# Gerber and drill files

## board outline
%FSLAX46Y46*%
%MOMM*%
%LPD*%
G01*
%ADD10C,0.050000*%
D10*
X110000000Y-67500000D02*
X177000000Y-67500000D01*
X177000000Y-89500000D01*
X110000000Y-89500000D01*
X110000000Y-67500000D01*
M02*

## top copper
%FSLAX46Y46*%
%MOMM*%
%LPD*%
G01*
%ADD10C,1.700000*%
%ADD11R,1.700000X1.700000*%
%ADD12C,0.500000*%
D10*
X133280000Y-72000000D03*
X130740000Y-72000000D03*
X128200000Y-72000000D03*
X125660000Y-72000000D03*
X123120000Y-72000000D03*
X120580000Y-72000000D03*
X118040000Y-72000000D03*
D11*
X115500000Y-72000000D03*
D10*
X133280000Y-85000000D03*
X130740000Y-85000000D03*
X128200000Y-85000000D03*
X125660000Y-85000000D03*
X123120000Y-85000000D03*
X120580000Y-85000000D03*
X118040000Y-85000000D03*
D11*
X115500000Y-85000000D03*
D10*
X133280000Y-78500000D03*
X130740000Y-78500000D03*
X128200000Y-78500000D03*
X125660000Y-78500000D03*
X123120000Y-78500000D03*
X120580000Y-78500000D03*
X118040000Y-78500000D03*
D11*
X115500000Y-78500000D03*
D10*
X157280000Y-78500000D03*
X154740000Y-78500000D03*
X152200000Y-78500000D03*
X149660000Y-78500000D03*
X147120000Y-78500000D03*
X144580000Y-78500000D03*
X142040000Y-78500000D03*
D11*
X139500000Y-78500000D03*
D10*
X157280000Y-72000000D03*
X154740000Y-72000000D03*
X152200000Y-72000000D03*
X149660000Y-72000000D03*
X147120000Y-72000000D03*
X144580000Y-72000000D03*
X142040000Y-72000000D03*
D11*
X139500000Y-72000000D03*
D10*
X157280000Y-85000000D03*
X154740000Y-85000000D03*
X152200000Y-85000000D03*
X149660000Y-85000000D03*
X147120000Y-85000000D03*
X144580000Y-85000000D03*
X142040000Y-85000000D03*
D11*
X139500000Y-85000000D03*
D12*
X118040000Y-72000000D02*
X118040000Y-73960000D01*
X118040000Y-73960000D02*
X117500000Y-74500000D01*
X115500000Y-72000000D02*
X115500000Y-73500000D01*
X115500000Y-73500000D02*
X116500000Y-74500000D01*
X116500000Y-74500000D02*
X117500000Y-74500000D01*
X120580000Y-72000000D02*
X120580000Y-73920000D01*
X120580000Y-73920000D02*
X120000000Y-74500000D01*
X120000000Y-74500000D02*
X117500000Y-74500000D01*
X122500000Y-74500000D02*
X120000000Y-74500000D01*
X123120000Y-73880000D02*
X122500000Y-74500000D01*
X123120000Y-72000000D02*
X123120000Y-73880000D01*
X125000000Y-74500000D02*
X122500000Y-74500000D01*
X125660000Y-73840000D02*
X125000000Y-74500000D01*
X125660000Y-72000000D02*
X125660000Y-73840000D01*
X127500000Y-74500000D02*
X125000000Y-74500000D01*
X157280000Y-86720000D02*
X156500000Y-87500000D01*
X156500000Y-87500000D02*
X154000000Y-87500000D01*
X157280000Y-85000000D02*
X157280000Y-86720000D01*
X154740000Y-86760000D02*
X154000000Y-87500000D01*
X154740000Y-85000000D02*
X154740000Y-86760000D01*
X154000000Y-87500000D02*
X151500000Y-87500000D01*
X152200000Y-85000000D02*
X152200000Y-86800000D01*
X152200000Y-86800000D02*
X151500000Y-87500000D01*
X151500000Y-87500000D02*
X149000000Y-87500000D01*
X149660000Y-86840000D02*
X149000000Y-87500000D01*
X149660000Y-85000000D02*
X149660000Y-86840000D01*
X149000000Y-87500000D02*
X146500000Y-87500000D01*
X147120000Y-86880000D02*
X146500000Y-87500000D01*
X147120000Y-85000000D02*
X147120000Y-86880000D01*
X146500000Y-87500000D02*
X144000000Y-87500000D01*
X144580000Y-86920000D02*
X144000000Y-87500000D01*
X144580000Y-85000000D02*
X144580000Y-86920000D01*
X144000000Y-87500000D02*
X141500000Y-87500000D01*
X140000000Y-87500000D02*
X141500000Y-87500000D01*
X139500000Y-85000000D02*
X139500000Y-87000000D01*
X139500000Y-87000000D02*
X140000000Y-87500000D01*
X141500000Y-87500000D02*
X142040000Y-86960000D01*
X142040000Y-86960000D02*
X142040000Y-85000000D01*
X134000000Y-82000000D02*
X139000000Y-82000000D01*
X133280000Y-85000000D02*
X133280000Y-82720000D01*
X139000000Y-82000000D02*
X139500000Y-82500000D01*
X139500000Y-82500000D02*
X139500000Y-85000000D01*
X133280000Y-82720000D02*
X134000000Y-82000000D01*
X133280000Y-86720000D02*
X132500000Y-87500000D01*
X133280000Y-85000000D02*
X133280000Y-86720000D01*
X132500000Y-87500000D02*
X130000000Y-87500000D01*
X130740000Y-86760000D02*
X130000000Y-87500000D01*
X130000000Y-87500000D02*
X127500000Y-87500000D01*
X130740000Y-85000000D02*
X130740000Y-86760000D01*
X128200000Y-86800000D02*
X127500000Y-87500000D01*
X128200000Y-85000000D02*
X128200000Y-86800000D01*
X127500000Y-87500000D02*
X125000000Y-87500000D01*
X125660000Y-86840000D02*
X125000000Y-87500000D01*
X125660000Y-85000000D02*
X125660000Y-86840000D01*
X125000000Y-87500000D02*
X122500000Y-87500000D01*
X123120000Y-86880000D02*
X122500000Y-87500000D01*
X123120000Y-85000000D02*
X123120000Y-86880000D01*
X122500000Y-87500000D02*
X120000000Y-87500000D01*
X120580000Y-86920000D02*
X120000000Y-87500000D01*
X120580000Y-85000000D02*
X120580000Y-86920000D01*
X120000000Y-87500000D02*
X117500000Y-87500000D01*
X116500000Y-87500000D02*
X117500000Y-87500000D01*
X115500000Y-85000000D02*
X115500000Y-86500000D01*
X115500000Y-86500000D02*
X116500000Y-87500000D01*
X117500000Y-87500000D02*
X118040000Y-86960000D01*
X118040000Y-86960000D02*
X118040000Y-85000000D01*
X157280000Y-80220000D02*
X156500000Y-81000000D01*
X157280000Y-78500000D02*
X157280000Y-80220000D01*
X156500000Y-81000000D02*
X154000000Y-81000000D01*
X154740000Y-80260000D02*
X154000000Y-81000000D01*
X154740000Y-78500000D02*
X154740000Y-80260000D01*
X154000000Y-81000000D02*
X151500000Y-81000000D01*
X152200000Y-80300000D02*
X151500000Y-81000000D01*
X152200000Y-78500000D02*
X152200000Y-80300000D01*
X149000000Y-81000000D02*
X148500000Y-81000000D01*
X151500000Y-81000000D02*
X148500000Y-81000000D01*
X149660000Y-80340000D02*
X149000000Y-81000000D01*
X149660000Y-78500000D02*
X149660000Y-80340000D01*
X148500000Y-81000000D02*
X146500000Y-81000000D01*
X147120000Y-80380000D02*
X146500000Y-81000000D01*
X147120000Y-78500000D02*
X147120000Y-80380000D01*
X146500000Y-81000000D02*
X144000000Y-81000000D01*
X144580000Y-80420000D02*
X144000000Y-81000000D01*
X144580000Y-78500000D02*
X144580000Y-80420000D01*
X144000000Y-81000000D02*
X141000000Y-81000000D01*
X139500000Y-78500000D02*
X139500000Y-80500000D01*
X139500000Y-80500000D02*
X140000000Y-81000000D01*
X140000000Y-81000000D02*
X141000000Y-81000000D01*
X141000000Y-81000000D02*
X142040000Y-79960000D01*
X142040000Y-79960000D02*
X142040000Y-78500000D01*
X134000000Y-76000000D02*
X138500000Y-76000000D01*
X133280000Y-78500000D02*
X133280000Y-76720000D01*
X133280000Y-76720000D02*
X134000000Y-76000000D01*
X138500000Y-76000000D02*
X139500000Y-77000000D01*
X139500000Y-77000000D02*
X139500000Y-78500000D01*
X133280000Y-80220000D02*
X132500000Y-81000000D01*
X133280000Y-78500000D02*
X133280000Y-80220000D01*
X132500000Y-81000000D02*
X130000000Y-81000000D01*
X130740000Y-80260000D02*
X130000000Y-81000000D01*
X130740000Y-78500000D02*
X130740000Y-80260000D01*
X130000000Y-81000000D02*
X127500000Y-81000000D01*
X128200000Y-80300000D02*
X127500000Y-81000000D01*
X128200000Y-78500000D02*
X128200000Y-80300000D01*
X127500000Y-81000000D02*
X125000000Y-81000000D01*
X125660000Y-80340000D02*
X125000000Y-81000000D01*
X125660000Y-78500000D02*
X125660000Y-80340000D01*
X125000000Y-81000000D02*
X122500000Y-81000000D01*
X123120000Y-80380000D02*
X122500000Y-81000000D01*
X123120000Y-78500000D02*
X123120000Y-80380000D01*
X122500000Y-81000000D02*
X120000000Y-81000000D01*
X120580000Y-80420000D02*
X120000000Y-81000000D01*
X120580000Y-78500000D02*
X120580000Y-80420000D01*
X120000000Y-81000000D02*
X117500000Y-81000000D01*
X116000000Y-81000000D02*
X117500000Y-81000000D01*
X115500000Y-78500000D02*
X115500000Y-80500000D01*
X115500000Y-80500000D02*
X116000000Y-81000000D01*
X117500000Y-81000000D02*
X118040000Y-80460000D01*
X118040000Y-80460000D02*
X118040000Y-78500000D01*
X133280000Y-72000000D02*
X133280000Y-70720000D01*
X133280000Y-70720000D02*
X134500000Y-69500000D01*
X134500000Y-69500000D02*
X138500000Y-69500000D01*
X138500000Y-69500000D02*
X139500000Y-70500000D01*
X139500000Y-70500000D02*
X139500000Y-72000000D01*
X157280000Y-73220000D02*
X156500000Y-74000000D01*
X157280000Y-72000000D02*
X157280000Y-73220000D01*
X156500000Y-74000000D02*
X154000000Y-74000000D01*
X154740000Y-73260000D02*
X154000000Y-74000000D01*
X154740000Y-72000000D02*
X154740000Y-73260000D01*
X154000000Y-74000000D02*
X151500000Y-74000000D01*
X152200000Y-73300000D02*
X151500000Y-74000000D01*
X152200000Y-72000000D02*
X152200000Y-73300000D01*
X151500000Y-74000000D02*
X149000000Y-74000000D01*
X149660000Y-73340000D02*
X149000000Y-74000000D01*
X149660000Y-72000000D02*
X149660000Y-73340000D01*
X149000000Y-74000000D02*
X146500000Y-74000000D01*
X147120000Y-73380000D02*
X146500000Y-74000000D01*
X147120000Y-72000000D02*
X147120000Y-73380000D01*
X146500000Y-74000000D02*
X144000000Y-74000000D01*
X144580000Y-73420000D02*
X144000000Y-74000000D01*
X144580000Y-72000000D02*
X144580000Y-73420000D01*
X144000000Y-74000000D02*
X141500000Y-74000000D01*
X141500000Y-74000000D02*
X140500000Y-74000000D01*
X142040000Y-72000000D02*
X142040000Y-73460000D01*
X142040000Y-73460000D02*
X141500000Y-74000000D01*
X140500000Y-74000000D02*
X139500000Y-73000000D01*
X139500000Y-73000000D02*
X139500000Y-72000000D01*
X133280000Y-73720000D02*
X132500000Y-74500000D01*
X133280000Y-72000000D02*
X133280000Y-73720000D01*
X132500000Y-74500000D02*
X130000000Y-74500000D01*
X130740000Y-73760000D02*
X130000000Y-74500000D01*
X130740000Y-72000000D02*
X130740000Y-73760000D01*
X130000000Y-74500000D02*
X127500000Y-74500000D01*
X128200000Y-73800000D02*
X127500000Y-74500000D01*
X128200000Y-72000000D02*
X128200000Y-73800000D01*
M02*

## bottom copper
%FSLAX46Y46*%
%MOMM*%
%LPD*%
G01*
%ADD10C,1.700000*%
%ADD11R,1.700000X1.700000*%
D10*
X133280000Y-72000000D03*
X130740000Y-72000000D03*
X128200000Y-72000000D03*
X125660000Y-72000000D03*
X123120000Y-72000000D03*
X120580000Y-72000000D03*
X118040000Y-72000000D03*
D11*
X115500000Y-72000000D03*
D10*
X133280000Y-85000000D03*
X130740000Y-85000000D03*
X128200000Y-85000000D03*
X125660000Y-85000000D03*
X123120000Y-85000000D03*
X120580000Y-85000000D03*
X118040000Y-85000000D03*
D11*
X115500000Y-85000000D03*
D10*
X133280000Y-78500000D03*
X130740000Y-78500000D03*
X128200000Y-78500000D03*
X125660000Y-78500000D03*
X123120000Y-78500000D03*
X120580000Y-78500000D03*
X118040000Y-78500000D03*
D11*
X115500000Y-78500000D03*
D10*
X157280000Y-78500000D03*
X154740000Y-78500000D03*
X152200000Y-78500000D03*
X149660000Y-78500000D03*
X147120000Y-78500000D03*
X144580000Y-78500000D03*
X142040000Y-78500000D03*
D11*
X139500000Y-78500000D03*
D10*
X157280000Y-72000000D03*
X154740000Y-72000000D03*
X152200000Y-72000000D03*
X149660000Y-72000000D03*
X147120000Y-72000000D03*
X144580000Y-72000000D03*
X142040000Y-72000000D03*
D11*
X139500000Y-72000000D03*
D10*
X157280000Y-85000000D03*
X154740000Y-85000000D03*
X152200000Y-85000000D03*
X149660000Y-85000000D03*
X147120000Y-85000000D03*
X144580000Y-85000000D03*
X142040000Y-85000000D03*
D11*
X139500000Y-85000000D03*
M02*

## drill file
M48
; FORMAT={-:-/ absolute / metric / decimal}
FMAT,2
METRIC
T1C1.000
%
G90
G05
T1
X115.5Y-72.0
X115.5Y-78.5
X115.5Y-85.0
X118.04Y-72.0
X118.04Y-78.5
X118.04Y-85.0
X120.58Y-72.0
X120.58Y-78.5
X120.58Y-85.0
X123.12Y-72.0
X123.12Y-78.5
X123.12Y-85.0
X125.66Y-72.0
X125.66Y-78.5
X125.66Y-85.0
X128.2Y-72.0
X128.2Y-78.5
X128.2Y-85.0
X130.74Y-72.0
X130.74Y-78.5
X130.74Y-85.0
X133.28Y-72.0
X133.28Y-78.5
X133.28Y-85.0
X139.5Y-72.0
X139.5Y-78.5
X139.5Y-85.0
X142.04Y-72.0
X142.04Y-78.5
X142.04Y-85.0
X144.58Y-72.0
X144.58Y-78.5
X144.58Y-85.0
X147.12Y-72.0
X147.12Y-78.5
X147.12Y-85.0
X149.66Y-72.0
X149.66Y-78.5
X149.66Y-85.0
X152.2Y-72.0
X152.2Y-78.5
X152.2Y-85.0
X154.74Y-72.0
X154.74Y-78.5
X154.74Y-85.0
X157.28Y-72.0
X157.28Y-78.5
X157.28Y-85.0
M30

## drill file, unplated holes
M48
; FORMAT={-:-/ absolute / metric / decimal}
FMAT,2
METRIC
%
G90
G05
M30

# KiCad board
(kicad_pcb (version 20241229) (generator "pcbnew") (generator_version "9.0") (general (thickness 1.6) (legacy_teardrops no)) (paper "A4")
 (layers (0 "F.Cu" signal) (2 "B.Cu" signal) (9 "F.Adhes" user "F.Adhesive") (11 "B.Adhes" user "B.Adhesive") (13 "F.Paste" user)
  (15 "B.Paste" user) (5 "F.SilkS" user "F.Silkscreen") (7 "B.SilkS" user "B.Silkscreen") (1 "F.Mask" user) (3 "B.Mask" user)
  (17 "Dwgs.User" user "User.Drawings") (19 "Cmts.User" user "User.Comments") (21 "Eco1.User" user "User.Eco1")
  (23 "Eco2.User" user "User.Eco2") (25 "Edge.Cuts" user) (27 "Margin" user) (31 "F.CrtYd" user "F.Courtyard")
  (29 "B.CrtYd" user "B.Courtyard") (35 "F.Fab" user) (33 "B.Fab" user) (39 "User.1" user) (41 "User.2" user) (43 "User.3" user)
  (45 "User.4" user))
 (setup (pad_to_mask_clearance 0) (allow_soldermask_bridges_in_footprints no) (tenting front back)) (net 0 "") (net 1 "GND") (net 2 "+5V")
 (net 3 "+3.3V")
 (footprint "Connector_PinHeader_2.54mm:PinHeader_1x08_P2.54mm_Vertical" (layer "F.Cu") (at 139.5 78.5 90)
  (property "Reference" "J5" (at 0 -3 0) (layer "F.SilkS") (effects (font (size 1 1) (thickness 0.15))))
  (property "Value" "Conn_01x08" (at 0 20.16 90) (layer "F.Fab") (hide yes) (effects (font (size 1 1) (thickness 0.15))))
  (pad "1" thru_hole rect (at 0 0 90) (size 1.7 1.7) (drill 1) (layers "*.Cu" "*.Mask") (remove_unused_layers no) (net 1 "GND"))
  (pad "2" thru_hole circle (at 0 2.54 90) (size 1.7 1.7) (drill 1) (layers "*.Cu" "*.Mask") (remove_unused_layers no) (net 1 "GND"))
  (pad "3" thru_hole circle (at 0 5.08 90) (size 1.7 1.7) (drill 1) (layers "*.Cu" "*.Mask") (remove_unused_layers no) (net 1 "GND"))
  (pad "4" thru_hole circle (at 0 7.62 90) (size 1.7 1.7) (drill 1) (layers "*.Cu" "*.Mask") (remove_unused_layers no) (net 1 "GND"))
  (pad "5" thru_hole circle (at 0 10.16 90) (size 1.7 1.7) (drill 1) (layers "*.Cu" "*.Mask") (remove_unused_layers no) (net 1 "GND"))
  (pad "6" thru_hole circle (at 0 12.7 90) (size 1.7 1.7) (drill 1) (layers "*.Cu" "*.Mask") (remove_unused_layers no) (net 1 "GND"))
  (pad "7" thru_hole circle (at 0 15.24 90) (size 1.7 1.7) (drill 1) (layers "*.Cu" "*.Mask") (remove_unused_layers no) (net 1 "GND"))
  (pad "8" thru_hole circle (at 0 17.78 90) (size 1.7 1.7) (drill 1) (layers "*.Cu" "*.Mask") (remove_unused_layers no) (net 1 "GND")))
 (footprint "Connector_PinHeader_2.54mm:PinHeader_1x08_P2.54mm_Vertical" (layer "F.Cu") (at 115.5 85 90)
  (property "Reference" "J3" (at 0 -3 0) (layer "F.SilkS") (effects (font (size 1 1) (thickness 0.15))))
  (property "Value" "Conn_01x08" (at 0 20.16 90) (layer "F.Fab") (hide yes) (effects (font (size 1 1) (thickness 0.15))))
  (pad "1" thru_hole rect (at 0 0 90) (size 1.7 1.7) (drill 1) (layers "*.Cu" "*.Mask") (remove_unused_layers no) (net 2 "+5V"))
  (pad "2" thru_hole circle (at 0 2.54 90) (size 1.7 1.7) (drill 1) (layers "*.Cu" "*.Mask") (remove_unused_layers no) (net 2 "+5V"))
  (pad "3" thru_hole circle (at 0 5.08 90) (size 1.7 1.7) (drill 1) (layers "*.Cu" "*.Mask") (remove_unused_layers no) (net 2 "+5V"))
  (pad "4" thru_hole circle (at 0 7.62 90) (size 1.7 1.7) (drill 1) (layers "*.Cu" "*.Mask") (remove_unused_layers no) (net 2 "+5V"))
  (pad "5" thru_hole circle (at 0 10.16 90) (size 1.7 1.7) (drill 1) (layers "*.Cu" "*.Mask") (remove_unused_layers no) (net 2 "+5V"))
  (pad "6" thru_hole circle (at 0 12.7 90) (size 1.7 1.7) (drill 1) (layers "*.Cu" "*.Mask") (remove_unused_layers no) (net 2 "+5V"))
  (pad "7" thru_hole circle (at 0 15.24 90) (size 1.7 1.7) (drill 1) (layers "*.Cu" "*.Mask") (remove_unused_layers no) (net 2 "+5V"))
  (pad "8" thru_hole circle (at 0 17.78 90) (size 1.7 1.7) (drill 1) (layers "*.Cu" "*.Mask") (remove_unused_layers no) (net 2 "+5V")))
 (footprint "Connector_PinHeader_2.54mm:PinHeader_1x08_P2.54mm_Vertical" (layer "F.Cu") (at 139.5 85 90)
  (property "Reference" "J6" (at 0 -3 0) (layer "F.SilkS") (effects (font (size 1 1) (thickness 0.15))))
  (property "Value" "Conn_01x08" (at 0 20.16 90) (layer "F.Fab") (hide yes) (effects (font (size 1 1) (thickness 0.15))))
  (pad "1" thru_hole rect (at 0 0 90) (size 1.7 1.7) (drill 1) (layers "*.Cu" "*.Mask") (remove_unused_layers no) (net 2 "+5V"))
  (pad "2" thru_hole circle (at 0 2.54 90) (size 1.7 1.7) (drill 1) (layers "*.Cu" "*.Mask") (remove_unused_layers no) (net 2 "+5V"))
  (pad "3" thru_hole circle (at 0 5.08 90) (size 1.7 1.7) (drill 1) (layers "*.Cu" "*.Mask") (remove_unused_layers no) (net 2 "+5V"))
  (pad "4" thru_hole circle (at 0 7.62 90) (size 1.7 1.7) (drill 1) (layers "*.Cu" "*.Mask") (remove_unused_layers no) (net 2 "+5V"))
  (pad "5" thru_hole circle (at 0 10.16 90) (size 1.7 1.7) (drill 1) (layers "*.Cu" "*.Mask") (remove_unused_layers no) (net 2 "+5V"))
  (pad "6" thru_hole circle (at 0 12.7 90) (size 1.7 1.7) (drill 1) (layers "*.Cu" "*.Mask") (remove_unused_layers no) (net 2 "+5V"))
  (pad "7" thru_hole circle (at 0 15.24 90) (size 1.7 1.7) (drill 1) (layers "*.Cu" "*.Mask") (remove_unused_layers no) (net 2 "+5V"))
  (pad "8" thru_hole circle (at 0 17.78 90) (size 1.7 1.7) (drill 1) (layers "*.Cu" "*.Mask") (remove_unused_layers no) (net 2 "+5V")))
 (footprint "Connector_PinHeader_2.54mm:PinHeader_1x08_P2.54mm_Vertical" (layer "F.Cu") (at 115.5 72 90)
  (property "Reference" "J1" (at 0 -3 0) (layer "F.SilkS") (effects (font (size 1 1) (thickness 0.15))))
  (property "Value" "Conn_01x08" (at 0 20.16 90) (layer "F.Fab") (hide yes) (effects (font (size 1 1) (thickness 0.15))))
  (pad "1" thru_hole rect (at 0 0 90) (size 1.7 1.7) (drill 1) (layers "*.Cu" "*.Mask") (remove_unused_layers no) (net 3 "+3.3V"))
  (pad "2" thru_hole circle (at 0 2.54 90) (size 1.7 1.7) (drill 1) (layers "*.Cu" "*.Mask") (remove_unused_layers no) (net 3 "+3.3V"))
  (pad "3" thru_hole circle (at 0 5.08 90) (size 1.7 1.7) (drill 1) (layers "*.Cu" "*.Mask") (remove_unused_layers no) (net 3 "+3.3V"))
  (pad "4" thru_hole circle (at 0 7.62 90) (size 1.7 1.7) (drill 1) (layers "*.Cu" "*.Mask") (remove_unused_layers no) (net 3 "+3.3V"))
  (pad "5" thru_hole circle (at 0 10.16 90) (size 1.7 1.7) (drill 1) (layers "*.Cu" "*.Mask") (remove_unused_layers no) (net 3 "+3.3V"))
  (pad "6" thru_hole circle (at 0 12.7 90) (size 1.7 1.7) (drill 1) (layers "*.Cu" "*.Mask") (remove_unused_layers no) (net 3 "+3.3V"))
  (pad "7" thru_hole circle (at 0 15.24 90) (size 1.7 1.7) (drill 1) (layers "*.Cu" "*.Mask") (remove_unused_layers no) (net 3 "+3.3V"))
  (pad "8" thru_hole circle (at 0 17.78 90) (size 1.7 1.7) (drill 1) (layers "*.Cu" "*.Mask") (remove_unused_layers no) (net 3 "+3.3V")))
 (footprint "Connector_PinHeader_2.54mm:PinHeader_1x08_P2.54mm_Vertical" (layer "F.Cu") (at 139.5 72 90)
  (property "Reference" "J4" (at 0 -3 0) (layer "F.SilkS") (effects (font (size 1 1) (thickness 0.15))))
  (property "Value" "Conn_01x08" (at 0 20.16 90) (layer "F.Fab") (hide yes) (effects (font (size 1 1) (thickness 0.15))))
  (pad "1" thru_hole rect (at 0 0 90) (size 1.7 1.7) (drill 1) (layers "*.Cu" "*.Mask") (remove_unused_layers no) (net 3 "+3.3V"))
  (pad "2" thru_hole circle (at 0 2.54 90) (size 1.7 1.7) (drill 1) (layers "*.Cu" "*.Mask") (remove_unused_layers no) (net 3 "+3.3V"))
  (pad "3" thru_hole circle (at 0 5.08 90) (size 1.7 1.7) (drill 1) (layers "*.Cu" "*.Mask") (remove_unused_layers no) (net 3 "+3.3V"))
  (pad "4" thru_hole circle (at 0 7.62 90) (size 1.7 1.7) (drill 1) (layers "*.Cu" "*.Mask") (remove_unused_layers no) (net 3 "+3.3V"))
  (pad "5" thru_hole circle (at 0 10.16 90) (size 1.7 1.7) (drill 1) (layers "*.Cu" "*.Mask") (remove_unused_layers no) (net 3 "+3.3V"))
  (pad "6" thru_hole circle (at 0 12.7 90) (size 1.7 1.7) (drill 1) (layers "*.Cu" "*.Mask") (remove_unused_layers no) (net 3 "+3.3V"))
  (pad "7" thru_hole circle (at 0 15.24 90) (size 1.7 1.7) (drill 1) (layers "*.Cu" "*.Mask") (remove_unused_layers no) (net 3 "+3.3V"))
  (pad "8" thru_hole circle (at 0 17.78 90) (size 1.7 1.7) (drill 1) (layers "*.Cu" "*.Mask") (remove_unused_layers no) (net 3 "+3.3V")))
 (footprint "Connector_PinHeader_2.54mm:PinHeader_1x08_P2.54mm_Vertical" (layer "F.Cu") (at 115.5 78.5 90)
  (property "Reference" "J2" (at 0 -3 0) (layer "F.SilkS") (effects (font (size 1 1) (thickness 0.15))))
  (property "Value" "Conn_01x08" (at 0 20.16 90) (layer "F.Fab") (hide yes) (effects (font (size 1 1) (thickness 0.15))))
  (pad "1" thru_hole rect (at 0 0 90) (size 1.7 1.7) (drill 1) (layers "*.Cu" "*.Mask") (remove_unused_layers no) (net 1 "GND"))
  (pad "2" thru_hole circle (at 0 2.54 90) (size 1.7 1.7) (drill 1) (layers "*.Cu" "*.Mask") (remove_unused_layers no) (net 1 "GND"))
  (pad "3" thru_hole circle (at 0 5.08 90) (size 1.7 1.7) (drill 1) (layers "*.Cu" "*.Mask") (remove_unused_layers no) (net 1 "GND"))
  (pad "4" thru_hole circle (at 0 7.62 90) (size 1.7 1.7) (drill 1) (layers "*.Cu" "*.Mask") (remove_unused_layers no) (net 1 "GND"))
  (pad "5" thru_hole circle (at 0 10.16 90) (size 1.7 1.7) (drill 1) (layers "*.Cu" "*.Mask") (remove_unused_layers no) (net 1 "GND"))
  (pad "6" thru_hole circle (at 0 12.7 90) (size 1.7 1.7) (drill 1) (layers "*.Cu" "*.Mask") (remove_unused_layers no) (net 1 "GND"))
  (pad "7" thru_hole circle (at 0 15.24 90) (size 1.7 1.7) (drill 1) (layers "*.Cu" "*.Mask") (remove_unused_layers no) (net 1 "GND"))
  (pad "8" thru_hole circle (at 0 17.78 90) (size 1.7 1.7) (drill 1) (layers "*.Cu" "*.Mask") (remove_unused_layers no) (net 1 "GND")))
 (gr_rect (start 110 67.5) (end 177 89.5) (stroke (width 0.05) (type default)) (fill no) (layer "Edge.Cuts"))
 (segment (start 130.74 72) (end 130.74 73.76) (width 0.5) (layer "F.Cu") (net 3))
 (segment (start 125 74.5) (end 122.5 74.5) (width 0.5) (layer "F.Cu") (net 3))
 (segment (start 152.2 73.3) (end 151.5 74) (width 0.5) (layer "F.Cu") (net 3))
 (segment (start 144.58 73.42) (end 144 74) (width 0.5) (layer "F.Cu") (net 3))
 (segment (start 125.66 73.84) (end 125 74.5) (width 0.5) (layer "F.Cu") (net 3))
 (segment (start 133.28 73.72) (end 132.5 74.5) (width 0.5) (layer "F.Cu") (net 3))
 (segment (start 142.04 72) (end 142.04 73.46) (width 0.5) (layer "F.Cu") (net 3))
 (segment (start 149.66 73.34) (end 149 74) (width 0.5) (layer "F.Cu") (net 3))
 (segment (start 152.2 72) (end 152.2 73.3) (width 0.5) (layer "F.Cu") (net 3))
 (segment (start 122.5 74.5) (end 120 74.5) (width 0.5) (layer "F.Cu") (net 3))
 (segment (start 141.5 74) (end 140.5 74) (width 0.5) (layer "F.Cu") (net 3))
 (segment (start 139.5 70.5) (end 139.5 72) (width 0.5) (layer "F.Cu") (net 3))
 (segment (start 118.04 73.96) (end 117.5 74.5) (width 0.5) (layer "F.Cu") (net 3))
 (segment (start 133.28 70.72) (end 134.5 69.5) (width 0.5) (layer "F.Cu") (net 3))
 (segment (start 140.5 74) (end 139.5 73) (width 0.5) (layer "F.Cu") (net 3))
 (segment (start 147.12 73.38) (end 146.5 74) (width 0.5) (layer "F.Cu") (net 3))
 (segment (start 132.5 74.5) (end 130 74.5) (width 0.5) (layer "F.Cu") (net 3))
 (segment (start 157.28 72) (end 157.28 73.22) (width 0.5) (layer "F.Cu") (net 3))
 (segment (start 154.74 73.26) (end 154 74) (width 0.5) (layer "F.Cu") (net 3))
 (segment (start 115.5 73.5) (end 116.5 74.5) (width 0.5) (layer "F.Cu") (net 3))
 (segment (start 133.28 72) (end 133.28 73.72) (width 0.5) (layer "F.Cu") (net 3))
 (segment (start 127.5 74.5) (end 125 74.5) (width 0.5) (layer "F.Cu") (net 3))
 (segment (start 123.12 73.88) (end 122.5 74.5) (width 0.5) (layer "F.Cu") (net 3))
 (segment (start 146.5 74) (end 144 74) (width 0.5) (layer "F.Cu") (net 3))
 (segment (start 120 74.5) (end 117.5 74.5) (width 0.5) (layer "F.Cu") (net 3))
 (segment (start 120.58 73.92) (end 120 74.5) (width 0.5) (layer "F.Cu") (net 3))
 (segment (start 115.5 72) (end 115.5 73.5) (width 0.5) (layer "F.Cu") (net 3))
 (segment (start 154 74) (end 151.5 74) (width 0.5) (layer "F.Cu") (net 3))
 (segment (start 128.2 73.8) (end 127.5 74.5) (width 0.5) (layer "F.Cu") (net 3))
 (segment (start 154.74 72) (end 154.74 73.26) (width 0.5) (layer "F.Cu") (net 3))
 (segment (start 133.28 72) (end 133.28 70.72) (width 0.5) (layer "F.Cu") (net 3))
 (segment (start 120.58 72) (end 120.58 73.92) (width 0.5) (layer "F.Cu") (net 3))
 (segment (start 149 74) (end 146.5 74) (width 0.5) (layer "F.Cu") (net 3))
 (segment (start 116.5 74.5) (end 117.5 74.5) (width 0.5) (layer "F.Cu") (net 3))
 (segment (start 123.12 72) (end 123.12 73.88) (width 0.5) (layer "F.Cu") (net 3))
 (segment (start 151.5 74) (end 149 74) (width 0.5) (layer "F.Cu") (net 3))
 (segment (start 156.5 74) (end 154 74) (width 0.5) (layer "F.Cu") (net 3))
 (segment (start 118.04 72) (end 118.04 73.96) (width 0.5) (layer "F.Cu") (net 3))
 (segment (start 130.74 73.76) (end 130 74.5) (width 0.5) (layer "F.Cu") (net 3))
 (segment (start 139.5 73) (end 139.5 72) (width 0.5) (layer "F.Cu") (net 3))
 (segment (start 128.2 72) (end 128.2 73.8) (width 0.5) (layer "F.Cu") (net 3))
 (segment (start 147.12 72) (end 147.12 73.38) (width 0.5) (layer "F.Cu") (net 3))
 (segment (start 130 74.5) (end 127.5 74.5) (width 0.5) (layer "F.Cu") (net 3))
 (segment (start 125.66 72) (end 125.66 73.84) (width 0.5) (layer "F.Cu") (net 3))
 (segment (start 144 74) (end 141.5 74) (width 0.5) (layer "F.Cu") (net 3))
 (segment (start 134.5 69.5) (end 138.5 69.5) (width 0.5) (layer "F.Cu") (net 3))
 (segment (start 142.04 73.46) (end 141.5 74) (width 0.5) (layer "F.Cu") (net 3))
 (segment (start 144.58 72) (end 144.58 73.42) (width 0.5) (layer "F.Cu") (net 3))
 (segment (start 149.66 72) (end 149.66 73.34) (width 0.5) (layer "F.Cu") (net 3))
 (segment (start 157.28 73.22) (end 156.5 74) (width 0.5) (layer "F.Cu") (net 3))
 (segment (start 138.5 69.5) (end 139.5 70.5) (width 0.5) (layer "F.Cu") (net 3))
 (segment (start 142.04 79.96) (end 142.04 78.5) (width 0.5) (layer "F.Cu") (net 1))
 (segment (start 147.12 78.5) (end 147.12 80.38) (width 0.5) (layer "F.Cu") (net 1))
 (segment (start 141 81) (end 142.04 79.96) (width 0.5) (layer "F.Cu") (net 1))
 (segment (start 128.2 80.3) (end 127.5 81) (width 0.5) (layer "F.Cu") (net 1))
 (segment (start 122.5 81) (end 120 81) (width 0.5) (layer "F.Cu") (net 1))
 (segment (start 146.5 81) (end 144 81) (width 0.5) (layer "F.Cu") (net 1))
 (segment (start 144.58 80.42) (end 144 81) (width 0.5) (layer "F.Cu") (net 1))
 (segment (start 125.66 78.5) (end 125.66 80.34) (width 0.5) (layer "F.Cu") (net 1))
 (segment (start 133.28 76.72) (end 134 76) (width 0.5) (layer "F.Cu") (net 1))
 (segment (start 115.5 78.5) (end 115.5 80.5) (width 0.5) (layer "F.Cu") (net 1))
 (segment (start 138.5 76) (end 139.5 77) (width 0.5) (layer "F.Cu") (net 1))
 (segment (start 123.12 80.38) (end 122.5 81) (width 0.5) (layer "F.Cu") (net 1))
 (segment (start 133.28 78.5) (end 133.28 80.22) (width 0.5) (layer "F.Cu") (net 1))
 (segment (start 127.5 81) (end 125 81) (width 0.5) (layer "F.Cu") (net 1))
 (segment (start 149 81) (end 148.5 81) (width 0.5) (layer "F.Cu") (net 1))
 (segment (start 130.74 80.26) (end 130 81) (width 0.5) (layer "F.Cu") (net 1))
 (segment (start 130.74 78.5) (end 130.74 80.26) (width 0.5) (layer "F.Cu") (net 1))
 (segment (start 152.2 78.5) (end 152.2 80.3) (width 0.5) (layer "F.Cu") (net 1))
 (segment (start 133.28 80.22) (end 132.5 81) (width 0.5) (layer "F.Cu") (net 1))
 (segment (start 123.12 78.5) (end 123.12 80.38) (width 0.5) (layer "F.Cu") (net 1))
 (segment (start 151.5 81) (end 148.5 81) (width 0.5) (layer "F.Cu") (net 1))
 (segment (start 140 81) (end 141 81) (width 0.5) (layer "F.Cu") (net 1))
 (segment (start 125 81) (end 122.5 81) (width 0.5) (layer "F.Cu") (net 1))
 (segment (start 148.5 81) (end 146.5 81) (width 0.5) (layer "F.Cu") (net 1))
 (segment (start 120.58 78.5) (end 120.58 80.42) (width 0.5) (layer "F.Cu") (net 1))
 (segment (start 157.28 80.22) (end 156.5 81) (width 0.5) (layer "F.Cu") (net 1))
 (segment (start 156.5 81) (end 154 81) (width 0.5) (layer "F.Cu") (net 1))
 (segment (start 115.5 80.5) (end 116 81) (width 0.5) (layer "F.Cu") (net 1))
 (segment (start 130 81) (end 127.5 81) (width 0.5) (layer "F.Cu") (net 1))
 (segment (start 144.58 78.5) (end 144.58 80.42) (width 0.5) (layer "F.Cu") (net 1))
 (segment (start 120 81) (end 117.5 81) (width 0.5) (layer "F.Cu") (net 1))
 (segment (start 154 81) (end 151.5 81) (width 0.5) (layer "F.Cu") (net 1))
 (segment (start 152.2 80.3) (end 151.5 81) (width 0.5) (layer "F.Cu") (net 1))
 (segment (start 132.5 81) (end 130 81) (width 0.5) (layer "F.Cu") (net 1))
 (segment (start 116 81) (end 117.5 81) (width 0.5) (layer "F.Cu") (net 1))
 (segment (start 144 81) (end 141 81) (width 0.5) (layer "F.Cu") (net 1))
 (segment (start 139.5 78.5) (end 139.5 80.5) (width 0.5) (layer "F.Cu") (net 1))
 (segment (start 118.04 80.46) (end 118.04 78.5) (width 0.5) (layer "F.Cu") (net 1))
 (segment (start 149.66 80.34) (end 149 81) (width 0.5) (layer "F.Cu") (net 1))
 (segment (start 125.66 80.34) (end 125 81) (width 0.5) (layer "F.Cu") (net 1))
 (segment (start 134 76) (end 138.5 76) (width 0.5) (layer "F.Cu") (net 1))
 (segment (start 154.74 80.26) (end 154 81) (width 0.5) (layer "F.Cu") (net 1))
 (segment (start 157.28 78.5) (end 157.28 80.22) (width 0.5) (layer "F.Cu") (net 1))
 (segment (start 117.5 81) (end 118.04 80.46) (width 0.5) (layer "F.Cu") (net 1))
 (segment (start 154.74 78.5) (end 154.74 80.26) (width 0.5) (layer "F.Cu") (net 1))
 (segment (start 133.28 78.5) (end 133.28 76.72) (width 0.5) (layer "F.Cu") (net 1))
 (segment (start 128.2 78.5) (end 128.2 80.3) (width 0.5) (layer "F.Cu") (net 1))
 (segment (start 149.66 78.5) (end 149.66 80.34) (width 0.5) (layer "F.Cu") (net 1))
 (segment (start 120.58 80.42) (end 120 81) (width 0.5) (layer "F.Cu") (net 1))
 (segment (start 139.5 77) (end 139.5 78.5) (width 0.5) (layer "F.Cu") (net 1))
 (segment (start 147.12 80.38) (end 146.5 81) (width 0.5) (layer "F.Cu") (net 1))
 (segment (start 139.5 80.5) (end 140 81) (width 0.5) (layer "F.Cu") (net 1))
 (segment (start 117.5 87.5) (end 118.04 86.96) (width 0.5) (layer "F.Cu") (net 2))
 (segment (start 125.66 86.84) (end 125 87.5) (width 0.5) (layer "F.Cu") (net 2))
 (segment (start 125 87.5) (end 122.5 87.5) (width 0.5) (layer "F.Cu") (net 2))
 (segment (start 154.74 86.76) (end 154 87.5) (width 0.5) (layer "F.Cu") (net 2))
 (segment (start 140 87.5) (end 141.5 87.5) (width 0.5) (layer "F.Cu") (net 2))
 (segment (start 118.04 86.96) (end 118.04 85) (width 0.5) (layer "F.Cu") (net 2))
 (segment (start 154.74 85) (end 154.74 86.76) (width 0.5) (layer "F.Cu") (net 2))
 (segment (start 115.5 85) (end 115.5 86.5) (width 0.5) (layer "F.Cu") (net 2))
 (segment (start 144 87.5) (end 141.5 87.5) (width 0.5) (layer "F.Cu") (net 2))
 (segment (start 132.5 87.5) (end 130 87.5) (width 0.5) (layer "F.Cu") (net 2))
 (segment (start 152.2 86.8) (end 151.5 87.5) (width 0.5) (layer "F.Cu") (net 2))
 (segment (start 133.28 85) (end 133.28 86.72) (width 0.5) (layer "F.Cu") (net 2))
 (segment (start 146.5 87.5) (end 144 87.5) (width 0.5) (layer "F.Cu") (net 2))
 (segment (start 123.12 86.88) (end 122.5 87.5) (width 0.5) (layer "F.Cu") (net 2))
 (segment (start 149 87.5) (end 146.5 87.5) (width 0.5) (layer "F.Cu") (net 2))
 (segment (start 147.12 85) (end 147.12 86.88) (width 0.5) (layer "F.Cu") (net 2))
 (segment (start 120.58 86.92) (end 120 87.5) (width 0.5) (layer "F.Cu") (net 2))
 (segment (start 133.28 85) (end 133.28 82.72) (width 0.5) (layer "F.Cu") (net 2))
 (segment (start 127.5 87.5) (end 125 87.5) (width 0.5) (layer "F.Cu") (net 2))
 (segment (start 125.66 85) (end 125.66 86.84) (width 0.5) (layer "F.Cu") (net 2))
 (segment (start 157.28 85) (end 157.28 86.72) (width 0.5) (layer "F.Cu") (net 2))
 (segment (start 128.2 85) (end 128.2 86.8) (width 0.5) (layer "F.Cu") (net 2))
 (segment (start 139 82) (end 139.5 82.5) (width 0.5) (layer "F.Cu") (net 2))
 (segment (start 157.28 86.72) (end 156.5 87.5) (width 0.5) (layer "F.Cu") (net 2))
 (segment (start 154 87.5) (end 151.5 87.5) (width 0.5) (layer "F.Cu") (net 2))
 (segment (start 147.12 86.88) (end 146.5 87.5) (width 0.5) (layer "F.Cu") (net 2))
 (segment (start 130.74 85) (end 130.74 86.76) (width 0.5) (layer "F.Cu") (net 2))
 (segment (start 139.5 87) (end 140 87.5) (width 0.5) (layer "F.Cu") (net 2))
 (segment (start 128.2 86.8) (end 127.5 87.5) (width 0.5) (layer "F.Cu") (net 2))
 (segment (start 133.28 82.72) (end 134 82) (width 0.5) (layer "F.Cu") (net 2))
 (segment (start 123.12 85) (end 123.12 86.88) (width 0.5) (layer "F.Cu") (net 2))
 (segment (start 144.58 85) (end 144.58 86.92) (width 0.5) (layer "F.Cu") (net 2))
 (segment (start 120.58 85) (end 120.58 86.92) (width 0.5) (layer "F.Cu") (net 2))
 (segment (start 149.66 85) (end 149.66 86.84) (width 0.5) (layer "F.Cu") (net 2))
 (segment (start 144.58 86.92) (end 144 87.5) (width 0.5) (layer "F.Cu") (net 2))
 (segment (start 130.74 86.76) (end 130 87.5) (width 0.5) (layer "F.Cu") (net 2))
 (segment (start 122.5 87.5) (end 120 87.5) (width 0.5) (layer "F.Cu") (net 2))
 (segment (start 156.5 87.5) (end 154 87.5) (width 0.5) (layer "F.Cu") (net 2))
 (segment (start 116.5 87.5) (end 117.5 87.5) (width 0.5) (layer "F.Cu") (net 2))
 (segment (start 134 82) (end 139 82) (width 0.5) (layer "F.Cu") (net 2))
 (segment (start 139.5 82.5) (end 139.5 85) (width 0.5) (layer "F.Cu") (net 2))
 (segment (start 152.2 85) (end 152.2 86.8) (width 0.5) (layer "F.Cu") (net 2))
 (segment (start 120 87.5) (end 117.5 87.5) (width 0.5) (layer "F.Cu") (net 2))
 (segment (start 130 87.5) (end 127.5 87.5) (width 0.5) (layer "F.Cu") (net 2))
 (segment (start 141.5 87.5) (end 142.04 86.96) (width 0.5) (layer "F.Cu") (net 2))
 (segment (start 133.28 86.72) (end 132.5 87.5) (width 0.5) (layer "F.Cu") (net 2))
 (segment (start 151.5 87.5) (end 149 87.5) (width 0.5) (layer "F.Cu") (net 2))
 (segment (start 142.04 86.96) (end 142.04 85) (width 0.5) (layer "F.Cu") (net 2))
 (segment (start 149.66 86.84) (end 149 87.5) (width 0.5) (layer "F.Cu") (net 2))
 (segment (start 139.5 85) (end 139.5 87) (width 0.5) (layer "F.Cu") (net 2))
 (segment (start 115.5 86.5) (end 116.5 87.5) (width 0.5) (layer "F.Cu") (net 2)))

